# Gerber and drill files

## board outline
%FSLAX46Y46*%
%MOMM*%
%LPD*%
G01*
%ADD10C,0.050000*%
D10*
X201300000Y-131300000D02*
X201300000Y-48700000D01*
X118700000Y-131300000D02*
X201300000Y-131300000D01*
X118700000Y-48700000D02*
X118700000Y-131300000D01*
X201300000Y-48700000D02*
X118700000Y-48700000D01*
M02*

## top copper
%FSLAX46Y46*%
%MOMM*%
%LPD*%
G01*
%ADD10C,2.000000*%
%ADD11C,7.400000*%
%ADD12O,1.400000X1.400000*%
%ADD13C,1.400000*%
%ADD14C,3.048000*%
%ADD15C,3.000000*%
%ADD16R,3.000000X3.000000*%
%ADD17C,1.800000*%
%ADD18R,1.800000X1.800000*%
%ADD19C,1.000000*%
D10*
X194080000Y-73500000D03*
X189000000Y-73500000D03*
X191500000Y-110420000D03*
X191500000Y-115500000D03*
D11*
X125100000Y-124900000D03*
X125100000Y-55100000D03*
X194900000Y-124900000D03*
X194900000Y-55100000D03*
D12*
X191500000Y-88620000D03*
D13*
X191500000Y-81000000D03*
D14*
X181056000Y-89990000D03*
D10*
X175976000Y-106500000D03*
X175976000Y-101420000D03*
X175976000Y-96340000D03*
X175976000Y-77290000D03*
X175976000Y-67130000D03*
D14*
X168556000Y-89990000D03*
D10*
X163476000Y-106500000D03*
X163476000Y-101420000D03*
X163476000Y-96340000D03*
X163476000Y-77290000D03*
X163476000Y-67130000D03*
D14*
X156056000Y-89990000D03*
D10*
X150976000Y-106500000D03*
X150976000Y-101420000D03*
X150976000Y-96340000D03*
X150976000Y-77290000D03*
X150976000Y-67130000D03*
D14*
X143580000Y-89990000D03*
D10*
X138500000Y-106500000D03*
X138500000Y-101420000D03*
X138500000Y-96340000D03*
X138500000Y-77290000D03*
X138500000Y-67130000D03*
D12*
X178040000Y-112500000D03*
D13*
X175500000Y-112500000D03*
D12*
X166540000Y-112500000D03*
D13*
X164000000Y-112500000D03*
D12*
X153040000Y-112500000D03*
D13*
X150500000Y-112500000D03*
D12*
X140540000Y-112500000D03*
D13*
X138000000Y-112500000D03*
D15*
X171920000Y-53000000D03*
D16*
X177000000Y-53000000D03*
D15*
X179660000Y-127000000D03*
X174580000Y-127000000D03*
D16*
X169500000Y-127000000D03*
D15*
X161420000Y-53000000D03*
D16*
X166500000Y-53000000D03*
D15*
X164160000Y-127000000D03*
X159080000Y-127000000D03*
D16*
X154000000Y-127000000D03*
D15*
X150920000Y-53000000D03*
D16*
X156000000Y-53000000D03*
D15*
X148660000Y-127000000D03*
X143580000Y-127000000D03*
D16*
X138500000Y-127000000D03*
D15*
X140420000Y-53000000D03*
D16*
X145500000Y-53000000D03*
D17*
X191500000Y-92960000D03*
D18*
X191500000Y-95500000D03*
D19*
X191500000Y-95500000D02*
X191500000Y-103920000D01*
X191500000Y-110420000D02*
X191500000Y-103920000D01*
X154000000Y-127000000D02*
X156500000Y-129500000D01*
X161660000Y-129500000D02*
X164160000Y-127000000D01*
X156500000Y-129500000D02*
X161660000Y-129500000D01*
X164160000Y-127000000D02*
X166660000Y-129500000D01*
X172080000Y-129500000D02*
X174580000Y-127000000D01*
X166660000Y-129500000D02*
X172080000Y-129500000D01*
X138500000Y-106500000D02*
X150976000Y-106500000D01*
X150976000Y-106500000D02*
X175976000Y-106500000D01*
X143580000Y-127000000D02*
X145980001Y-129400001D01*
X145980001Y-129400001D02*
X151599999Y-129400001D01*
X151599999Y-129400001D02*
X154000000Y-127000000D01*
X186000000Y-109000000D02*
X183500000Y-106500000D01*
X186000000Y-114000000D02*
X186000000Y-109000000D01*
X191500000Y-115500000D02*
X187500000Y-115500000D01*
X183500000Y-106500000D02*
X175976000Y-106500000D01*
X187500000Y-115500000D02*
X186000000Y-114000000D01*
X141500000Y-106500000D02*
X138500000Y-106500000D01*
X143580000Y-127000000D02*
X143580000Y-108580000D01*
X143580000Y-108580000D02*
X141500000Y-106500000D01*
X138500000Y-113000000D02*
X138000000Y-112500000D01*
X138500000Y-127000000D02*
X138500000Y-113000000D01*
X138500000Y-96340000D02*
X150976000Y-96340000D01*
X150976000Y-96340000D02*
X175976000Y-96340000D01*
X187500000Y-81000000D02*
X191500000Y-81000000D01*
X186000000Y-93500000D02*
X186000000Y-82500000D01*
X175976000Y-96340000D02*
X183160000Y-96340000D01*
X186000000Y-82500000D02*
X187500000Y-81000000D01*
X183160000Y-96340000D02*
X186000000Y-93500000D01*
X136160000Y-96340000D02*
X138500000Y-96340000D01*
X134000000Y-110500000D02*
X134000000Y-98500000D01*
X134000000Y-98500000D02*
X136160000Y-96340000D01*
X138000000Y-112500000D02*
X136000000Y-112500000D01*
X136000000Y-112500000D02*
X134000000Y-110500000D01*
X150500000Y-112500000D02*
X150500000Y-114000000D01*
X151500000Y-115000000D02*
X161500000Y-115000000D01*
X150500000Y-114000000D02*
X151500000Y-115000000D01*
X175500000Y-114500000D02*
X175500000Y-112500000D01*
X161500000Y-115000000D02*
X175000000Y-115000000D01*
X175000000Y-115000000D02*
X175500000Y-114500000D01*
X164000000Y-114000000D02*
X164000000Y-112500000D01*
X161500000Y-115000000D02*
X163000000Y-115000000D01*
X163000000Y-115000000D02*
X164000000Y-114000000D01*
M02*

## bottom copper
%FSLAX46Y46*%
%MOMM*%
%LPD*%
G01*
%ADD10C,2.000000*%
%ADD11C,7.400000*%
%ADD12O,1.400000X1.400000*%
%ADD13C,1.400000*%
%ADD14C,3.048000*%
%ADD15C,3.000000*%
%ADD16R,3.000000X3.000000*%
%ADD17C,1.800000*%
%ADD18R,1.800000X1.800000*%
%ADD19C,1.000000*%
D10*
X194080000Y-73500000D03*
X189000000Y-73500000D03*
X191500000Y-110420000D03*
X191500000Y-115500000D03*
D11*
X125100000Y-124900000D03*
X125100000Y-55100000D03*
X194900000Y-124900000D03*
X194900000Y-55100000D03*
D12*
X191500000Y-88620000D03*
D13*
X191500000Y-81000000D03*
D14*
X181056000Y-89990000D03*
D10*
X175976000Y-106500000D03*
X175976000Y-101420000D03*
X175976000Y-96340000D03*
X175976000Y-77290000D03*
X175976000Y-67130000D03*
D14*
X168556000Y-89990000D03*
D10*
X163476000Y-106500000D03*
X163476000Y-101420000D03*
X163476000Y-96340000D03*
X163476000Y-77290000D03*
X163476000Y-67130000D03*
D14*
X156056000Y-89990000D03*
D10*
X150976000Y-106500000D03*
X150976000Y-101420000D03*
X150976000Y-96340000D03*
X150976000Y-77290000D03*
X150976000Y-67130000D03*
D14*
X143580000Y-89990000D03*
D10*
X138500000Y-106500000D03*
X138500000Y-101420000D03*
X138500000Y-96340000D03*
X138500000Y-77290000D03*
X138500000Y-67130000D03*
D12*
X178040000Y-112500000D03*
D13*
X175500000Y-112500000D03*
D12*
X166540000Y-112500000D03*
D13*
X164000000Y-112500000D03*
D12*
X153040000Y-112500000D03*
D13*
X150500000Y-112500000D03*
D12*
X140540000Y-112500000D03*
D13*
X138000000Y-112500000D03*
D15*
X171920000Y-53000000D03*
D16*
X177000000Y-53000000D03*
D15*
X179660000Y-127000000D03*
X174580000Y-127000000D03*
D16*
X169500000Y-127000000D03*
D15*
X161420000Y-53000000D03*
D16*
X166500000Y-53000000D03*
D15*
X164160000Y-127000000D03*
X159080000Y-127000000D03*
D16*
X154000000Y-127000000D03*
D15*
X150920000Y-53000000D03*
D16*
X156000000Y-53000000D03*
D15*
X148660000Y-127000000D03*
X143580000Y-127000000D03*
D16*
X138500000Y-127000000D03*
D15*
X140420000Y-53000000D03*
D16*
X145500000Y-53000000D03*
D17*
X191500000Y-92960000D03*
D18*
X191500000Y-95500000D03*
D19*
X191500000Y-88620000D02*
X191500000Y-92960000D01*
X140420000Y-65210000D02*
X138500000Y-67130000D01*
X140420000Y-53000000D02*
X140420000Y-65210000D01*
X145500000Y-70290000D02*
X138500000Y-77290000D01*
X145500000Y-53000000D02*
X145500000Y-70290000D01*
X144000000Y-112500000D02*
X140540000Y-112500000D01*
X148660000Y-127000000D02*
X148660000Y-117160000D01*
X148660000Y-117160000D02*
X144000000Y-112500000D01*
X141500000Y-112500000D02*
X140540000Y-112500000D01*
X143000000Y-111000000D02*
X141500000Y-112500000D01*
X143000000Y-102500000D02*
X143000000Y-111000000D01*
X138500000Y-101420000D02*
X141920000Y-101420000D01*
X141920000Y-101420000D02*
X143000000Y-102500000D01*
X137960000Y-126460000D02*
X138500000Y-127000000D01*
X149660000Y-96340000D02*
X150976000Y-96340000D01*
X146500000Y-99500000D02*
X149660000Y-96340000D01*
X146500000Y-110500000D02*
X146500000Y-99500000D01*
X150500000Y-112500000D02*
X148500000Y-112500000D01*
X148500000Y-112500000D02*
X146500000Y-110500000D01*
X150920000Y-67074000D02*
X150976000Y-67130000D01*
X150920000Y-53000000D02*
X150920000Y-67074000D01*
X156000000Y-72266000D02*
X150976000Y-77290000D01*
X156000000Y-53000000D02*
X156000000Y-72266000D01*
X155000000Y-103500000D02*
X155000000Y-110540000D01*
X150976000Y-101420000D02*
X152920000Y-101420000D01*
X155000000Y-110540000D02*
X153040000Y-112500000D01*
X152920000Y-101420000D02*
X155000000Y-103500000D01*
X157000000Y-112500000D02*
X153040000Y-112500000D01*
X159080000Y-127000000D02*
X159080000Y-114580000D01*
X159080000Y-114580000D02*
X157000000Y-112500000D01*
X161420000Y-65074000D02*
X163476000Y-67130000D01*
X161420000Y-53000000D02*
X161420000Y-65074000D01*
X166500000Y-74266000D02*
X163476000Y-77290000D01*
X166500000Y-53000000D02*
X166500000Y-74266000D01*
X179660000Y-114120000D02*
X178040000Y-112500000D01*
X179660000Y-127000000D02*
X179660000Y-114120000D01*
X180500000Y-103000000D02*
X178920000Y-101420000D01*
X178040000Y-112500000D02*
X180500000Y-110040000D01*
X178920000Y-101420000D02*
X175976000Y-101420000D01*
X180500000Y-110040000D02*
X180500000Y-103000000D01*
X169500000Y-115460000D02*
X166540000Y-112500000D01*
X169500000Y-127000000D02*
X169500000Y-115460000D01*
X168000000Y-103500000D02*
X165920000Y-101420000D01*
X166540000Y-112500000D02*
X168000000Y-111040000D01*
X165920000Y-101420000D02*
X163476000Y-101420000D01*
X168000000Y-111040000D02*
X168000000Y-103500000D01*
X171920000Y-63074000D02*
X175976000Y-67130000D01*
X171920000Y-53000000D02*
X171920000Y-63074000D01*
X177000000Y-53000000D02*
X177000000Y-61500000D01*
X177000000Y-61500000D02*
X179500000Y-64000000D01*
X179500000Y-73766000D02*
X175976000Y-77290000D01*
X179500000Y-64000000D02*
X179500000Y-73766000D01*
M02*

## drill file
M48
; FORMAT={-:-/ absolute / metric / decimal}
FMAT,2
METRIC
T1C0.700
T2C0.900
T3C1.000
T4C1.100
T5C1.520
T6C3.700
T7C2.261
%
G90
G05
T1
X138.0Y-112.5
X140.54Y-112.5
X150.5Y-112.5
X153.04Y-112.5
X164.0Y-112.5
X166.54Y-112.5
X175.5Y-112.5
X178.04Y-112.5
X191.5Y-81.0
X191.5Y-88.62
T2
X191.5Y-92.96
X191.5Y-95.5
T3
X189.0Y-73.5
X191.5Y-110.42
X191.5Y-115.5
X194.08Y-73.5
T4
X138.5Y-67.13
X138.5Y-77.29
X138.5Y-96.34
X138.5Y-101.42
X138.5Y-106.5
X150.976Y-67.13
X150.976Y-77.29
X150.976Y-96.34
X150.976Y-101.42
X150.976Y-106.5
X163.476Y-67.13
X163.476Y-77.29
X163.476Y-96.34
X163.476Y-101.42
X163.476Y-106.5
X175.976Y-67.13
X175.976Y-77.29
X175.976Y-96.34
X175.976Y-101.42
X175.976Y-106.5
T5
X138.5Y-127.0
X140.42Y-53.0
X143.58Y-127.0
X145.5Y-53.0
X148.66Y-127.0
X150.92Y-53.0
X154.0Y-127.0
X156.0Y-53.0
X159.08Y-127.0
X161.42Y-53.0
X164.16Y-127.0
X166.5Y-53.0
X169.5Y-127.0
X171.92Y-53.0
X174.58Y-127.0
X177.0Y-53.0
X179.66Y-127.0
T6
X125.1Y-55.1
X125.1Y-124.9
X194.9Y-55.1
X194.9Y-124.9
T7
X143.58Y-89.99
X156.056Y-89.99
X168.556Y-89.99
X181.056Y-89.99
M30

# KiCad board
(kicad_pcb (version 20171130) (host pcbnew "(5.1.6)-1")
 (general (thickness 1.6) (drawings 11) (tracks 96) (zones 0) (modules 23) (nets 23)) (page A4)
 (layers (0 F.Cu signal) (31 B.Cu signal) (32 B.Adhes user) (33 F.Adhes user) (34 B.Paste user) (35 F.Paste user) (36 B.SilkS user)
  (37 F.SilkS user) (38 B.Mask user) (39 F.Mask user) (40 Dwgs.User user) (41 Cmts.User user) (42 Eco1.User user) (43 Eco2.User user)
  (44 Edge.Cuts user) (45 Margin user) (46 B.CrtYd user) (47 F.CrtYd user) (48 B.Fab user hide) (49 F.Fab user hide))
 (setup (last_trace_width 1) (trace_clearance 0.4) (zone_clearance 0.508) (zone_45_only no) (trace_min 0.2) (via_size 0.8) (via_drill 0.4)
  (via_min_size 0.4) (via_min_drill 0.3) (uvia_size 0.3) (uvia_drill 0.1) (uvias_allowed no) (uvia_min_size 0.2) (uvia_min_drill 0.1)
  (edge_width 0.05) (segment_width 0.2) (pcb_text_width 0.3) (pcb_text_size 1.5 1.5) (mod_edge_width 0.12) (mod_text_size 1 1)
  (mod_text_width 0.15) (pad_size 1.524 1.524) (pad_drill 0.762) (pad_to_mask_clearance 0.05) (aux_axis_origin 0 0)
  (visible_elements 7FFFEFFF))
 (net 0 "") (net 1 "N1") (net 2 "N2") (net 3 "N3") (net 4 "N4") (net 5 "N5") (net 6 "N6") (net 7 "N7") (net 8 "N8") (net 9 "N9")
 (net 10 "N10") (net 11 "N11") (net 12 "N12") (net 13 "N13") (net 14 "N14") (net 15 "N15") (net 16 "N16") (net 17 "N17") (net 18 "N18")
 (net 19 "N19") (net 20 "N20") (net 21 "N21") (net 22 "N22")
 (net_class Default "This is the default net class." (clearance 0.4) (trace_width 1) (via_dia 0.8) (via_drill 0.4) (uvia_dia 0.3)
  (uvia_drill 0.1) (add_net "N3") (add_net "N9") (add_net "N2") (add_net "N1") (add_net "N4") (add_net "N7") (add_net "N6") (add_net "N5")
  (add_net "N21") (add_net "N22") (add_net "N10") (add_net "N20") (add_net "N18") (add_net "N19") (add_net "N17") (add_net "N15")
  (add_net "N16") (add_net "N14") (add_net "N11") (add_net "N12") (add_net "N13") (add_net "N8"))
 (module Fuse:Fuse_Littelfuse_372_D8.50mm (layer F.Cu) (at 189 73.5)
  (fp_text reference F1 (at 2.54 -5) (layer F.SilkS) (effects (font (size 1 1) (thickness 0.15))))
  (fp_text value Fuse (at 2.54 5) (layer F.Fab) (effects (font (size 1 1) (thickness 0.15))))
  (pad 2 thru_hole circle (at 5.08 0) (size 2 2) (drill 1) (layers *.Cu *.Mask) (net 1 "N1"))
  (pad 1 thru_hole circle (at 0 0) (size 2 2) (drill 1) (layers *.Cu *.Mask) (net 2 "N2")))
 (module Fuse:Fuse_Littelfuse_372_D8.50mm (layer F.Cu) (at 191.5 115.5 90)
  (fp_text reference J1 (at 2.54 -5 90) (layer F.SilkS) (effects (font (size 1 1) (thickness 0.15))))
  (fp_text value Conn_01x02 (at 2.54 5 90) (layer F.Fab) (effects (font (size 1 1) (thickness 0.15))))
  (pad 2 thru_hole circle (at 5.08 0 90) (size 2 2) (drill 1) (layers *.Cu *.Mask) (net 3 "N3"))
  (pad 1 thru_hole circle (at 0 0 90) (size 2 2) (drill 1) (layers *.Cu *.Mask) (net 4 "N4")))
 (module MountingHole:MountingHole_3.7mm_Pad (layer F.Cu) (at 125.1 124.9)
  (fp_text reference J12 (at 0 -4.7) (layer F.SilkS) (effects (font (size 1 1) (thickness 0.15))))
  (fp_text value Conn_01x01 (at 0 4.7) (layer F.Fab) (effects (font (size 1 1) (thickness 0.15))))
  (pad 1 thru_hole circle (at 0 0) (size 7.4 7.4) (drill 3.7) (layers *.Cu *.Mask) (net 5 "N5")))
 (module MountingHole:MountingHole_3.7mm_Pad (layer F.Cu) (at 125.1 55.1)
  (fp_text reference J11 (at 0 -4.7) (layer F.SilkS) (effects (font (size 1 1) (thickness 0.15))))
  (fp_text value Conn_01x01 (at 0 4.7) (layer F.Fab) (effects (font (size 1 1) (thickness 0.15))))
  (pad 1 thru_hole circle (at 0 0) (size 7.4 7.4) (drill 3.7) (layers *.Cu *.Mask) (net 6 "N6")))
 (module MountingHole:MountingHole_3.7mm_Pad (layer F.Cu) (at 194.9 124.9)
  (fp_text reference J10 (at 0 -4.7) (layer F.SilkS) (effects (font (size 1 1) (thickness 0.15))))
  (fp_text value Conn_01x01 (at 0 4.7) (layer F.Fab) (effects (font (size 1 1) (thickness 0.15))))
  (pad 1 thru_hole circle (at 0 0) (size 7.4 7.4) (drill 3.7) (layers *.Cu *.Mask) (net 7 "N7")))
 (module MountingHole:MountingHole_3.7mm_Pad (layer F.Cu) (at 194.9 55.1)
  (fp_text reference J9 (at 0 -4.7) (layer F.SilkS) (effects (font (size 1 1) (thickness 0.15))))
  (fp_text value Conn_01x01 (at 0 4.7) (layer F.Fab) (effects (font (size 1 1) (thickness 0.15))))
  (pad 1 thru_hole circle (at 0 0) (size 7.4 7.4) (drill 3.7) (layers *.Cu *.Mask) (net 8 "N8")))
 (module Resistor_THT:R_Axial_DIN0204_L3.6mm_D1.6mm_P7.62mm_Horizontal (layer F.Cu) (at 191.5 81 270)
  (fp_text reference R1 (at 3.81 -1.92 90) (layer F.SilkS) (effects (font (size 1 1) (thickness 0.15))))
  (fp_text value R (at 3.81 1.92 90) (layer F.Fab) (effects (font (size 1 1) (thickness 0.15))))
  (pad 2 thru_hole oval (at 7.62 0 270) (size 1.4 1.4) (drill 0.7) (layers *.Cu *.Mask) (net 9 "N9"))
  (pad 1 thru_hole circle (at 0 0 270) (size 1.4 1.4) (drill 0.7) (layers *.Cu *.Mask) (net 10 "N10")))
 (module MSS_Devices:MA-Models (layer F.Cu) (at 177.5 106.5 90)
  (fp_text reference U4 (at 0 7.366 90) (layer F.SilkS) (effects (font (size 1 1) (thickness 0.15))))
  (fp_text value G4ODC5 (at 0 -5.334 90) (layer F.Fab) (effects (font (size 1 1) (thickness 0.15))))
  (pad "" np_thru_hole circle (at 16.51 3.556 90) (size 3.048 3.048) (drill 2.2606) (layers *.Cu *.Mask))
  (pad 5 thru_hole circle (at 0 -1.524 90) (size 2 2) (drill 1.1) (layers *.Cu *.Mask) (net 4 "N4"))
  (pad 4 thru_hole circle (at 5.08 -1.524 90) (size 2 2) (drill 1.1) (layers *.Cu *.Mask) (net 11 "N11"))
  (pad 3 thru_hole circle (at 10.16 -1.524 90) (size 2 2) (drill 1.1) (layers *.Cu *.Mask) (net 10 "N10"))
  (pad 2 thru_hole circle (at 29.21 -1.524 90) (size 2 2) (drill 1.1) (layers *.Cu *.Mask) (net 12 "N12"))
  (pad 1 thru_hole circle (at 39.37 -1.524 90) (size 2 2) (drill 1.1) (layers *.Cu *.Mask) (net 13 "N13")))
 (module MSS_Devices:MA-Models (layer F.Cu) (at 165 106.5 90)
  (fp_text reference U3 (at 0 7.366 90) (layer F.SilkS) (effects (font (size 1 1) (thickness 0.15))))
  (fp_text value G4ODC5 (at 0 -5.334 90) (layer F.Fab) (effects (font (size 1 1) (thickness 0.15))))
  (pad "" np_thru_hole circle (at 16.51 3.556 90) (size 3.048 3.048) (drill 2.2606) (layers *.Cu *.Mask))
  (pad 5 thru_hole circle (at 0 -1.524 90) (size 2 2) (drill 1.1) (layers *.Cu *.Mask) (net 4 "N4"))
  (pad 4 thru_hole circle (at 5.08 -1.524 90) (size 2 2) (drill 1.1) (layers *.Cu *.Mask) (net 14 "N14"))
  (pad 3 thru_hole circle (at 10.16 -1.524 90) (size 2 2) (drill 1.1) (layers *.Cu *.Mask) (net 10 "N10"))
  (pad 2 thru_hole circle (at 29.21 -1.524 90) (size 2 2) (drill 1.1) (layers *.Cu *.Mask) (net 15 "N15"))
  (pad 1 thru_hole circle (at 39.37 -1.524 90) (size 2 2) (drill 1.1) (layers *.Cu *.Mask) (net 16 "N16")))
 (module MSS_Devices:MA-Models (layer F.Cu) (at 152.5 106.5 90)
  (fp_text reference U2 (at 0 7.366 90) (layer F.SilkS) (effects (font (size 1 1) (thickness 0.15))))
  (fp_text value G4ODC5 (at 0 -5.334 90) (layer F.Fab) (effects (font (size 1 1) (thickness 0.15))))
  (pad "" np_thru_hole circle (at 16.51 3.556 90) (size 3.048 3.048) (drill 2.2606) (layers *.Cu *.Mask))
  (pad 5 thru_hole circle (at 0 -1.524 90) (size 2 2) (drill 1.1) (layers *.Cu *.Mask) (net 4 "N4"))
  (pad 4 thru_hole circle (at 5.08 -1.524 90) (size 2 2) (drill 1.1) (layers *.Cu *.Mask) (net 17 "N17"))
  (pad 3 thru_hole circle (at 10.16 -1.524 90) (size 2 2) (drill 1.1) (layers *.Cu *.Mask) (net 10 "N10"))
  (pad 2 thru_hole circle (at 29.21 -1.524 90) (size 2 2) (drill 1.1) (layers *.Cu *.Mask) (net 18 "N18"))
  (pad 1 thru_hole circle (at 39.37 -1.524 90) (size 2 2) (drill 1.1) (layers *.Cu *.Mask) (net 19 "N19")))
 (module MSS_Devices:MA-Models (layer F.Cu) (at 140.024 106.5 90)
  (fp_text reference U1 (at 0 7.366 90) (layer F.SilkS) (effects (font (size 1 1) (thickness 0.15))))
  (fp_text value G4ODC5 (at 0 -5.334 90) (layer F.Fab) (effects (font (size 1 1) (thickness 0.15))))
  (pad "" np_thru_hole circle (at 16.51 3.556 90) (size 3.048 3.048) (drill 2.2606) (layers *.Cu *.Mask))
  (pad 5 thru_hole circle (at 0 -1.524 90) (size 2 2) (drill 1.1) (layers *.Cu *.Mask) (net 4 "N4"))
  (pad 4 thru_hole circle (at 5.08 -1.524 90) (size 2 2) (drill 1.1) (layers *.Cu *.Mask) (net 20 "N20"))
  (pad 3 thru_hole circle (at 10.16 -1.524 90) (size 2 2) (drill 1.1) (layers *.Cu *.Mask) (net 10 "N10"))
  (pad 2 thru_hole circle (at 29.21 -1.524 90) (size 2 2) (drill 1.1) (layers *.Cu *.Mask) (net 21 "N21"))
  (pad 1 thru_hole circle (at 39.37 -1.524 90) (size 2 2) (drill 1.1) (layers *.Cu *.Mask) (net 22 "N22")))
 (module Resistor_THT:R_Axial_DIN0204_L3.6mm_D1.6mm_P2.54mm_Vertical (layer F.Cu) (at 175.5 112.5)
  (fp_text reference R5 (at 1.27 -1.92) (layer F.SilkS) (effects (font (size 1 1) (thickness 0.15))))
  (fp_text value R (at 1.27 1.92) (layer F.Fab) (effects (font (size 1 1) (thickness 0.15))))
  (pad 2 thru_hole oval (at 2.54 0) (size 1.4 1.4) (drill 0.7) (layers *.Cu *.Mask) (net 11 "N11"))
  (pad 1 thru_hole circle (at 0 0) (size 1.4 1.4) (drill 0.7) (layers *.Cu *.Mask) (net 10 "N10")))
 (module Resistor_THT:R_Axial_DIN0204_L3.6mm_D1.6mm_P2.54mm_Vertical (layer F.Cu) (at 164 112.5)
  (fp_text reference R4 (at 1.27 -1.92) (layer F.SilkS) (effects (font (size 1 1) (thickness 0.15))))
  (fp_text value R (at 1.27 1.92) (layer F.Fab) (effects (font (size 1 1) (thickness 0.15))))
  (pad 2 thru_hole oval (at 2.54 0) (size 1.4 1.4) (drill 0.7) (layers *.Cu *.Mask) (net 14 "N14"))
  (pad 1 thru_hole circle (at 0 0) (size 1.4 1.4) (drill 0.7) (layers *.Cu *.Mask) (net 10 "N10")))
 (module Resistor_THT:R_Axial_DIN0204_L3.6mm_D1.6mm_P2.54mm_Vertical (layer F.Cu) (at 150.5 112.5)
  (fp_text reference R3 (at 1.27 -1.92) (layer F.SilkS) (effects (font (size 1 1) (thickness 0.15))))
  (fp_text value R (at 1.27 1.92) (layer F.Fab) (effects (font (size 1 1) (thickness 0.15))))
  (pad 2 thru_hole oval (at 2.54 0) (size 1.4 1.4) (drill 0.7) (layers *.Cu *.Mask) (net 17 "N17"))
  (pad 1 thru_hole circle (at 0 0) (size 1.4 1.4) (drill 0.7) (layers *.Cu *.Mask) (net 10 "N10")))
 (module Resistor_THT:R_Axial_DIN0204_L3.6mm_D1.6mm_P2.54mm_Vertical (layer F.Cu) (at 138 112.5)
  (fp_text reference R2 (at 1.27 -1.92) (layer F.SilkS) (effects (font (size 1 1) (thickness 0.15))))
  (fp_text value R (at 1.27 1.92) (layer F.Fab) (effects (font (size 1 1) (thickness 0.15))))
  (pad 2 thru_hole oval (at 2.54 0) (size 1.4 1.4) (drill 0.7) (layers *.Cu *.Mask) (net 20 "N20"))
  (pad 1 thru_hole circle (at 0 0) (size 1.4 1.4) (drill 0.7) (layers *.Cu *.Mask) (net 10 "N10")))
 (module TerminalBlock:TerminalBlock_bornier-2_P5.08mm (layer F.Cu) (at 177 53 180)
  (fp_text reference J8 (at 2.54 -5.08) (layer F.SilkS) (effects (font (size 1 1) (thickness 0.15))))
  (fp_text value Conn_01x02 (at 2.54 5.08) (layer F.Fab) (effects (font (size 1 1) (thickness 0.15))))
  (pad 2 thru_hole circle (at 5.08 0 180) (size 3 3) (drill 1.52) (layers *.Cu *.Mask) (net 13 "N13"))
  (pad 1 thru_hole rect (at 0 0 180) (size 3 3) (drill 1.52) (layers *.Cu *.Mask) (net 12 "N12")))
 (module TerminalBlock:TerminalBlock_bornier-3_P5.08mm (layer F.Cu) (at 169.5 127)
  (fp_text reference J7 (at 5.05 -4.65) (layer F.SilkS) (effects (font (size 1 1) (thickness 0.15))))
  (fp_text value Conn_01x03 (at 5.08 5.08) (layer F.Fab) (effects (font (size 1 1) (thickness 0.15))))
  (pad 3 thru_hole circle (at 10.16 0) (size 3 3) (drill 1.52) (layers *.Cu *.Mask) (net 11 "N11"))
  (pad 2 thru_hole circle (at 5.08 0) (size 3 3) (drill 1.52) (layers *.Cu *.Mask) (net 4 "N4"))
  (pad 1 thru_hole rect (at 0 0) (size 3 3) (drill 1.52) (layers *.Cu *.Mask) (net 14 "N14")))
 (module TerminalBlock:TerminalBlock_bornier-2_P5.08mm (layer F.Cu) (at 166.5 53 180)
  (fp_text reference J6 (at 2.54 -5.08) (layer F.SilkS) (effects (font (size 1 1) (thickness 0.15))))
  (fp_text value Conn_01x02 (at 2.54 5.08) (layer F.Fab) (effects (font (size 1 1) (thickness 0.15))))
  (pad 2 thru_hole circle (at 5.08 0 180) (size 3 3) (drill 1.52) (layers *.Cu *.Mask) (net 16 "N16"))
  (pad 1 thru_hole rect (at 0 0 180) (size 3 3) (drill 1.52) (layers *.Cu *.Mask) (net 15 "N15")))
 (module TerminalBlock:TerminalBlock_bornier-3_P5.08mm (layer F.Cu) (at 154 127)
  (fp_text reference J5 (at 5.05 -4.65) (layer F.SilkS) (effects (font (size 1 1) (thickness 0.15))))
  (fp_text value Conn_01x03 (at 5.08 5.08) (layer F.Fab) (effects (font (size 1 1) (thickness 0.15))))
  (pad 3 thru_hole circle (at 10.16 0) (size 3 3) (drill 1.52) (layers *.Cu *.Mask) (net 4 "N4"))
  (pad 2 thru_hole circle (at 5.08 0) (size 3 3) (drill 1.52) (layers *.Cu *.Mask) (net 17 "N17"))
  (pad 1 thru_hole rect (at 0 0) (size 3 3) (drill 1.52) (layers *.Cu *.Mask) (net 4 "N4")))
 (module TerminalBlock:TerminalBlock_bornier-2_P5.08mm (layer F.Cu) (at 156 53 180)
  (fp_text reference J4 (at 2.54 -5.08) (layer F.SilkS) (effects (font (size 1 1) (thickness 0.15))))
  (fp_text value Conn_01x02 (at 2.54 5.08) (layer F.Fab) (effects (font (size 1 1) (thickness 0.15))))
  (pad 2 thru_hole circle (at 5.08 0 180) (size 3 3) (drill 1.52) (layers *.Cu *.Mask) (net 19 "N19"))
  (pad 1 thru_hole rect (at 0 0 180) (size 3 3) (drill 1.52) (layers *.Cu *.Mask) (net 18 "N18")))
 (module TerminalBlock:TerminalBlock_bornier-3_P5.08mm (layer F.Cu) (at 138.5 127)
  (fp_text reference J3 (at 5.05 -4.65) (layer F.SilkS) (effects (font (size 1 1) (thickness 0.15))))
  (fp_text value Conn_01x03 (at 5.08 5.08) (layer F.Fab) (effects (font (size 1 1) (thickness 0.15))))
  (pad 3 thru_hole circle (at 10.16 0) (size 3 3) (drill 1.52) (layers *.Cu *.Mask) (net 20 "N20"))
  (pad 2 thru_hole circle (at 5.08 0) (size 3 3) (drill 1.52) (layers *.Cu *.Mask) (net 4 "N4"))
  (pad 1 thru_hole rect (at 0 0) (size 3 3) (drill 1.52) (layers *.Cu *.Mask) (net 10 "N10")))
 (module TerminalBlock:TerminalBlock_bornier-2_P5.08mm (layer F.Cu) (at 145.5 53 180)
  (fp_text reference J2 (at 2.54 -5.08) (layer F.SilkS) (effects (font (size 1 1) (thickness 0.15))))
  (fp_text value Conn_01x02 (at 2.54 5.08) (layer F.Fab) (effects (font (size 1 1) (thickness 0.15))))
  (pad 2 thru_hole circle (at 5.08 0 180) (size 3 3) (drill 1.52) (layers *.Cu *.Mask) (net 22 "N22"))
  (pad 1 thru_hole rect (at 0 0 180) (size 3 3) (drill 1.52) (layers *.Cu *.Mask) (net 21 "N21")))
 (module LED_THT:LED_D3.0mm (layer F.Cu) (at 191.5 95.5 90)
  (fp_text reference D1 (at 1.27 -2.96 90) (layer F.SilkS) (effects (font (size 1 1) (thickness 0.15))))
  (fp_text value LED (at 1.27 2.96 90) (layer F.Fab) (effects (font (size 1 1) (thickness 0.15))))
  (pad 2 thru_hole circle (at 2.54 0 90) (size 1.8 1.8) (drill 0.9) (layers *.Cu *.Mask) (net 9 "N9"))
  (pad 1 thru_hole rect (at 0 0 90) (size 1.8 1.8) (drill 0.9) (layers *.Cu *.Mask) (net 3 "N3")))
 (gr_line (start 201.3 131.3) (end 201.3 48.7) (layer Edge.Cuts) (width 0.05))
 (gr_line (start 118.7 131.3) (end 201.3 131.3) (layer Edge.Cuts) (width 0.05))
 (gr_line (start 118.7 48.7) (end 118.7 131.3) (layer Edge.Cuts) (width 0.05))
 (gr_line (start 201.3 48.7) (end 118.7 48.7) (layer Edge.Cuts) (width 0.05))
 (segment (start 191.5 88.62) (end 191.5 92.96) (width 1) (layer B.Cu) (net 9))
 (segment (start 191.5 95.5) (end 191.5 103.92) (width 1) (layer F.Cu) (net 3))
 (segment (start 191.5 110.42) (end 191.5 103.92) (width 1) (layer F.Cu) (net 3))
 (segment (start 154 127) (end 156.5 129.5) (width 1) (layer F.Cu) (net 4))
 (segment (start 161.66 129.5) (end 164.16 127) (width 1) (layer F.Cu) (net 4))
 (segment (start 156.5 129.5) (end 161.66 129.5) (width 1) (layer F.Cu) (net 4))
 (segment (start 164.16 127) (end 166.66 129.5) (width 1) (layer F.Cu) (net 4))
 (segment (start 172.08 129.5) (end 174.58 127) (width 1) (layer F.Cu) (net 4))
 (segment (start 166.66 129.5) (end 172.08 129.5) (width 1) (layer F.Cu) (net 4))
 (segment (start 138.5 106.5) (end 150.976 106.5) (width 1) (layer F.Cu) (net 4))
 (segment (start 150.976 106.5) (end 175.976 106.5) (width 1) (layer F.Cu) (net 4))
 (segment (start 143.58 127) (end 145.980001 129.400001) (width 1) (layer F.Cu) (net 4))
 (segment (start 145.980001 129.400001) (end 151.599999 129.400001) (width 1) (layer F.Cu) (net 4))
 (segment (start 151.599999 129.400001) (end 154 127) (width 1) (layer F.Cu) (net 4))
 (segment (start 186 109) (end 183.5 106.5) (width 1) (layer F.Cu) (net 4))
 (segment (start 186 114) (end 186 109) (width 1) (layer F.Cu) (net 4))
 (segment (start 191.5 115.5) (end 187.5 115.5) (width 1) (layer F.Cu) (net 4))
 (segment (start 183.5 106.5) (end 175.976 106.5) (width 1) (layer F.Cu) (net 4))
 (segment (start 187.5 115.5) (end 186 114) (width 1) (layer F.Cu) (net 4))
 (segment (start 141.5 106.5) (end 138.5 106.5) (width 1) (layer F.Cu) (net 4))
 (segment (start 143.58 127) (end 143.58 108.58) (width 1) (layer F.Cu) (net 4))
 (segment (start 143.58 108.58) (end 141.5 106.5) (width 1) (layer F.Cu) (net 4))
 (segment (start 140.42 65.21) (end 138.5 67.13) (width 1) (layer B.Cu) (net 22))
 (segment (start 140.42 53) (end 140.42 65.21) (width 1) (layer B.Cu) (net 22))
 (segment (start 145.5 70.29) (end 138.5 77.29) (width 1) (layer B.Cu) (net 21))
 (segment (start 145.5 53) (end 145.5 70.29) (width 1) (layer B.Cu) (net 21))
 (segment (start 144 112.5) (end 140.54 112.5) (width 1) (layer B.Cu) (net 20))
 (segment (start 148.66 127) (end 148.66 117.16) (width 1) (layer B.Cu) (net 20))
 (segment (start 148.66 117.16) (end 144 112.5) (width 1) (layer B.Cu) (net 20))
 (segment (start 141.5 112.5) (end 140.54 112.5) (width 1) (layer B.Cu) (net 20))
 (segment (start 143 111) (end 141.5 112.5) (width 1) (layer B.Cu) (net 20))
 (segment (start 143 102.5) (end 143 111) (width 1) (layer B.Cu) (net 20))
 (segment (start 138.5 101.42) (end 141.92 101.42) (width 1) (layer B.Cu) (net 20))
 (segment (start 141.92 101.42) (end 143 102.5) (width 1) (layer B.Cu) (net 20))
 (segment (start 137.96 126.46) (end 138.5 127) (width 1) (layer B.Cu) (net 10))
 (segment (start 138.5 113) (end 138 112.5) (width 1) (layer F.Cu) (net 10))
 (segment (start 138.5 127) (end 138.5 113) (width 1) (layer F.Cu) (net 10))
 (segment (start 138.5 96.34) (end 150.976 96.34) (width 1) (layer F.Cu) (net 10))
 (segment (start 150.976 96.34) (end 175.976 96.34) (width 1) (layer F.Cu) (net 10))
 (segment (start 187.5 81) (end 191.5 81) (width 1) (layer F.Cu) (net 10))
 (segment (start 186 93.5) (end 186 82.5) (width 1) (layer F.Cu) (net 10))
 (segment (start 175.976 96.34) (end 183.16 96.34) (width 1) (layer F.Cu) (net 10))
 (segment (start 186 82.5) (end 187.5 81) (width 1) (layer F.Cu) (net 10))
 (segment (start 183.16 96.34) (end 186 93.5) (width 1) (layer F.Cu) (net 10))
 (segment (start 136.16 96.34) (end 138.5 96.34) (width 1) (layer F.Cu) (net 10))
 (segment (start 134 110.5) (end 134 98.5) (width 1) (layer F.Cu) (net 10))
 (segment (start 134 98.5) (end 136.16 96.34) (width 1) (layer F.Cu) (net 10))
 (segment (start 138 112.5) (end 136 112.5) (width 1) (layer F.Cu) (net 10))
 (segment (start 136 112.5) (end 134 110.5) (width 1) (layer F.Cu) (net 10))
 (segment (start 150.5 112.5) (end 150.5 114) (width 1) (layer F.Cu) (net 10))
 (segment (start 151.5 115) (end 161.5 115) (width 1) (layer F.Cu) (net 10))
 (segment (start 150.5 114) (end 151.5 115) (width 1) (layer F.Cu) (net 10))
 (segment (start 175.5 114.5) (end 175.5 112.5) (width 1) (layer F.Cu) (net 10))
 (segment (start 161.5 115) (end 175 115) (width 1) (layer F.Cu) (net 10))
 (segment (start 175 115) (end 175.5 114.5) (width 1) (layer F.Cu) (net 10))
 (segment (start 164 114) (end 164 112.5) (width 1) (layer F.Cu) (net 10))
 (segment (start 161.5 115) (end 163 115) (width 1) (layer F.Cu) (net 10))
 (segment (start 163 115) (end 164 114) (width 1) (layer F.Cu) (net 10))
 (segment (start 149.66 96.34) (end 150.976 96.34) (width 1) (layer B.Cu) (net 10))
 (segment (start 146.5 99.5) (end 149.66 96.34) (width 1) (layer B.Cu) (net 10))
 (segment (start 146.5 110.5) (end 146.5 99.5) (width 1) (layer B.Cu) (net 10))
 (segment (start 150.5 112.5) (end 148.5 112.5) (width 1) (layer B.Cu) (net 10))
 (segment (start 148.5 112.5) (end 146.5 110.5) (width 1) (layer B.Cu) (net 10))
 (segment (start 150.92 67.074) (end 150.976 67.13) (width 1) (layer B.Cu) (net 19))
 (segment (start 150.92 53) (end 150.92 67.074) (width 1) (layer B.Cu) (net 19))
 (segment (start 156 72.266) (end 150.976 77.29) (width 1) (layer B.Cu) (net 18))
 (segment (start 156 53) (end 156 72.266) (width 1) (layer B.Cu) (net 18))
 (segment (start 155 103.5) (end 155 110.54) (width 1) (layer B.Cu) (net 17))
 (segment (start 150.976 101.42) (end 152.92 101.42) (width 1) (layer B.Cu) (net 17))
 (segment (start 155 110.54) (end 153.04 112.5) (width 1) (layer B.Cu) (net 17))
 (segment (start 152.92 101.42) (end 155 103.5) (width 1) (layer B.Cu) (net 17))
 (segment (start 157 112.5) (end 153.04 112.5) (width 1) (layer B.Cu) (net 17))
 (segment (start 159.08 127) (end 159.08 114.58) (width 1) (layer B.Cu) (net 17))
 (segment (start 159.08 114.58) (end 157 112.5) (width 1) (layer B.Cu) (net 17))
 (segment (start 161.42 65.074) (end 163.476 67.13) (width 1) (layer B.Cu) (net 16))
 (segment (start 161.42 53) (end 161.42 65.074) (width 1) (layer B.Cu) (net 16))
 (segment (start 166.5 74.266) (end 163.476 77.29) (width 1) (layer B.Cu) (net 15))
 (segment (start 166.5 53) (end 166.5 74.266) (width 1) (layer B.Cu) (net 15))
 (segment (start 179.66 114.12) (end 178.04 112.5) (width 1) (layer B.Cu) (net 11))
 (segment (start 179.66 127) (end 179.66 114.12) (width 1) (layer B.Cu) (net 11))
 (segment (start 180.5 103) (end 178.92 101.42) (width 1) (layer B.Cu) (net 11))
 (segment (start 178.04 112.5) (end 180.5 110.04) (width 1) (layer B.Cu) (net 11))
 (segment (start 178.92 101.42) (end 175.976 101.42) (width 1) (layer B.Cu) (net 11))
 (segment (start 180.5 110.04) (end 180.5 103) (width 1) (layer B.Cu) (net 11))
 (segment (start 169.5 115.46) (end 166.54 112.5) (width 1) (layer B.Cu) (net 14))
 (segment (start 169.5 127) (end 169.5 115.46) (width 1) (layer B.Cu) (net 14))
 (segment (start 168 103.5) (end 165.92 101.42) (width 1) (layer B.Cu) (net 14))
 (segment (start 166.54 112.5) (end 168 111.04) (width 1) (layer B.Cu) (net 14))
 (segment (start 165.92 101.42) (end 163.476 101.42) (width 1) (layer B.Cu) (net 14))
 (segment (start 168 111.04) (end 168 103.5) (width 1) (layer B.Cu) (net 14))
 (segment (start 171.92 63.074) (end 175.976 67.13) (width 1) (layer B.Cu) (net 13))
 (segment (start 171.92 53) (end 171.92 63.074) (width 1) (layer B.Cu) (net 13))
 (segment (start 177 53) (end 177 61.5) (width 1) (layer B.Cu) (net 12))
 (segment (start 177 61.5) (end 179.5 64) (width 1) (layer B.Cu) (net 12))
 (segment (start 179.5 73.766) (end 175.976 77.29) (width 1) (layer B.Cu) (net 12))
 (segment (start 179.5 64) (end 179.5 73.766) (width 1) (layer B.Cu) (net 12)))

